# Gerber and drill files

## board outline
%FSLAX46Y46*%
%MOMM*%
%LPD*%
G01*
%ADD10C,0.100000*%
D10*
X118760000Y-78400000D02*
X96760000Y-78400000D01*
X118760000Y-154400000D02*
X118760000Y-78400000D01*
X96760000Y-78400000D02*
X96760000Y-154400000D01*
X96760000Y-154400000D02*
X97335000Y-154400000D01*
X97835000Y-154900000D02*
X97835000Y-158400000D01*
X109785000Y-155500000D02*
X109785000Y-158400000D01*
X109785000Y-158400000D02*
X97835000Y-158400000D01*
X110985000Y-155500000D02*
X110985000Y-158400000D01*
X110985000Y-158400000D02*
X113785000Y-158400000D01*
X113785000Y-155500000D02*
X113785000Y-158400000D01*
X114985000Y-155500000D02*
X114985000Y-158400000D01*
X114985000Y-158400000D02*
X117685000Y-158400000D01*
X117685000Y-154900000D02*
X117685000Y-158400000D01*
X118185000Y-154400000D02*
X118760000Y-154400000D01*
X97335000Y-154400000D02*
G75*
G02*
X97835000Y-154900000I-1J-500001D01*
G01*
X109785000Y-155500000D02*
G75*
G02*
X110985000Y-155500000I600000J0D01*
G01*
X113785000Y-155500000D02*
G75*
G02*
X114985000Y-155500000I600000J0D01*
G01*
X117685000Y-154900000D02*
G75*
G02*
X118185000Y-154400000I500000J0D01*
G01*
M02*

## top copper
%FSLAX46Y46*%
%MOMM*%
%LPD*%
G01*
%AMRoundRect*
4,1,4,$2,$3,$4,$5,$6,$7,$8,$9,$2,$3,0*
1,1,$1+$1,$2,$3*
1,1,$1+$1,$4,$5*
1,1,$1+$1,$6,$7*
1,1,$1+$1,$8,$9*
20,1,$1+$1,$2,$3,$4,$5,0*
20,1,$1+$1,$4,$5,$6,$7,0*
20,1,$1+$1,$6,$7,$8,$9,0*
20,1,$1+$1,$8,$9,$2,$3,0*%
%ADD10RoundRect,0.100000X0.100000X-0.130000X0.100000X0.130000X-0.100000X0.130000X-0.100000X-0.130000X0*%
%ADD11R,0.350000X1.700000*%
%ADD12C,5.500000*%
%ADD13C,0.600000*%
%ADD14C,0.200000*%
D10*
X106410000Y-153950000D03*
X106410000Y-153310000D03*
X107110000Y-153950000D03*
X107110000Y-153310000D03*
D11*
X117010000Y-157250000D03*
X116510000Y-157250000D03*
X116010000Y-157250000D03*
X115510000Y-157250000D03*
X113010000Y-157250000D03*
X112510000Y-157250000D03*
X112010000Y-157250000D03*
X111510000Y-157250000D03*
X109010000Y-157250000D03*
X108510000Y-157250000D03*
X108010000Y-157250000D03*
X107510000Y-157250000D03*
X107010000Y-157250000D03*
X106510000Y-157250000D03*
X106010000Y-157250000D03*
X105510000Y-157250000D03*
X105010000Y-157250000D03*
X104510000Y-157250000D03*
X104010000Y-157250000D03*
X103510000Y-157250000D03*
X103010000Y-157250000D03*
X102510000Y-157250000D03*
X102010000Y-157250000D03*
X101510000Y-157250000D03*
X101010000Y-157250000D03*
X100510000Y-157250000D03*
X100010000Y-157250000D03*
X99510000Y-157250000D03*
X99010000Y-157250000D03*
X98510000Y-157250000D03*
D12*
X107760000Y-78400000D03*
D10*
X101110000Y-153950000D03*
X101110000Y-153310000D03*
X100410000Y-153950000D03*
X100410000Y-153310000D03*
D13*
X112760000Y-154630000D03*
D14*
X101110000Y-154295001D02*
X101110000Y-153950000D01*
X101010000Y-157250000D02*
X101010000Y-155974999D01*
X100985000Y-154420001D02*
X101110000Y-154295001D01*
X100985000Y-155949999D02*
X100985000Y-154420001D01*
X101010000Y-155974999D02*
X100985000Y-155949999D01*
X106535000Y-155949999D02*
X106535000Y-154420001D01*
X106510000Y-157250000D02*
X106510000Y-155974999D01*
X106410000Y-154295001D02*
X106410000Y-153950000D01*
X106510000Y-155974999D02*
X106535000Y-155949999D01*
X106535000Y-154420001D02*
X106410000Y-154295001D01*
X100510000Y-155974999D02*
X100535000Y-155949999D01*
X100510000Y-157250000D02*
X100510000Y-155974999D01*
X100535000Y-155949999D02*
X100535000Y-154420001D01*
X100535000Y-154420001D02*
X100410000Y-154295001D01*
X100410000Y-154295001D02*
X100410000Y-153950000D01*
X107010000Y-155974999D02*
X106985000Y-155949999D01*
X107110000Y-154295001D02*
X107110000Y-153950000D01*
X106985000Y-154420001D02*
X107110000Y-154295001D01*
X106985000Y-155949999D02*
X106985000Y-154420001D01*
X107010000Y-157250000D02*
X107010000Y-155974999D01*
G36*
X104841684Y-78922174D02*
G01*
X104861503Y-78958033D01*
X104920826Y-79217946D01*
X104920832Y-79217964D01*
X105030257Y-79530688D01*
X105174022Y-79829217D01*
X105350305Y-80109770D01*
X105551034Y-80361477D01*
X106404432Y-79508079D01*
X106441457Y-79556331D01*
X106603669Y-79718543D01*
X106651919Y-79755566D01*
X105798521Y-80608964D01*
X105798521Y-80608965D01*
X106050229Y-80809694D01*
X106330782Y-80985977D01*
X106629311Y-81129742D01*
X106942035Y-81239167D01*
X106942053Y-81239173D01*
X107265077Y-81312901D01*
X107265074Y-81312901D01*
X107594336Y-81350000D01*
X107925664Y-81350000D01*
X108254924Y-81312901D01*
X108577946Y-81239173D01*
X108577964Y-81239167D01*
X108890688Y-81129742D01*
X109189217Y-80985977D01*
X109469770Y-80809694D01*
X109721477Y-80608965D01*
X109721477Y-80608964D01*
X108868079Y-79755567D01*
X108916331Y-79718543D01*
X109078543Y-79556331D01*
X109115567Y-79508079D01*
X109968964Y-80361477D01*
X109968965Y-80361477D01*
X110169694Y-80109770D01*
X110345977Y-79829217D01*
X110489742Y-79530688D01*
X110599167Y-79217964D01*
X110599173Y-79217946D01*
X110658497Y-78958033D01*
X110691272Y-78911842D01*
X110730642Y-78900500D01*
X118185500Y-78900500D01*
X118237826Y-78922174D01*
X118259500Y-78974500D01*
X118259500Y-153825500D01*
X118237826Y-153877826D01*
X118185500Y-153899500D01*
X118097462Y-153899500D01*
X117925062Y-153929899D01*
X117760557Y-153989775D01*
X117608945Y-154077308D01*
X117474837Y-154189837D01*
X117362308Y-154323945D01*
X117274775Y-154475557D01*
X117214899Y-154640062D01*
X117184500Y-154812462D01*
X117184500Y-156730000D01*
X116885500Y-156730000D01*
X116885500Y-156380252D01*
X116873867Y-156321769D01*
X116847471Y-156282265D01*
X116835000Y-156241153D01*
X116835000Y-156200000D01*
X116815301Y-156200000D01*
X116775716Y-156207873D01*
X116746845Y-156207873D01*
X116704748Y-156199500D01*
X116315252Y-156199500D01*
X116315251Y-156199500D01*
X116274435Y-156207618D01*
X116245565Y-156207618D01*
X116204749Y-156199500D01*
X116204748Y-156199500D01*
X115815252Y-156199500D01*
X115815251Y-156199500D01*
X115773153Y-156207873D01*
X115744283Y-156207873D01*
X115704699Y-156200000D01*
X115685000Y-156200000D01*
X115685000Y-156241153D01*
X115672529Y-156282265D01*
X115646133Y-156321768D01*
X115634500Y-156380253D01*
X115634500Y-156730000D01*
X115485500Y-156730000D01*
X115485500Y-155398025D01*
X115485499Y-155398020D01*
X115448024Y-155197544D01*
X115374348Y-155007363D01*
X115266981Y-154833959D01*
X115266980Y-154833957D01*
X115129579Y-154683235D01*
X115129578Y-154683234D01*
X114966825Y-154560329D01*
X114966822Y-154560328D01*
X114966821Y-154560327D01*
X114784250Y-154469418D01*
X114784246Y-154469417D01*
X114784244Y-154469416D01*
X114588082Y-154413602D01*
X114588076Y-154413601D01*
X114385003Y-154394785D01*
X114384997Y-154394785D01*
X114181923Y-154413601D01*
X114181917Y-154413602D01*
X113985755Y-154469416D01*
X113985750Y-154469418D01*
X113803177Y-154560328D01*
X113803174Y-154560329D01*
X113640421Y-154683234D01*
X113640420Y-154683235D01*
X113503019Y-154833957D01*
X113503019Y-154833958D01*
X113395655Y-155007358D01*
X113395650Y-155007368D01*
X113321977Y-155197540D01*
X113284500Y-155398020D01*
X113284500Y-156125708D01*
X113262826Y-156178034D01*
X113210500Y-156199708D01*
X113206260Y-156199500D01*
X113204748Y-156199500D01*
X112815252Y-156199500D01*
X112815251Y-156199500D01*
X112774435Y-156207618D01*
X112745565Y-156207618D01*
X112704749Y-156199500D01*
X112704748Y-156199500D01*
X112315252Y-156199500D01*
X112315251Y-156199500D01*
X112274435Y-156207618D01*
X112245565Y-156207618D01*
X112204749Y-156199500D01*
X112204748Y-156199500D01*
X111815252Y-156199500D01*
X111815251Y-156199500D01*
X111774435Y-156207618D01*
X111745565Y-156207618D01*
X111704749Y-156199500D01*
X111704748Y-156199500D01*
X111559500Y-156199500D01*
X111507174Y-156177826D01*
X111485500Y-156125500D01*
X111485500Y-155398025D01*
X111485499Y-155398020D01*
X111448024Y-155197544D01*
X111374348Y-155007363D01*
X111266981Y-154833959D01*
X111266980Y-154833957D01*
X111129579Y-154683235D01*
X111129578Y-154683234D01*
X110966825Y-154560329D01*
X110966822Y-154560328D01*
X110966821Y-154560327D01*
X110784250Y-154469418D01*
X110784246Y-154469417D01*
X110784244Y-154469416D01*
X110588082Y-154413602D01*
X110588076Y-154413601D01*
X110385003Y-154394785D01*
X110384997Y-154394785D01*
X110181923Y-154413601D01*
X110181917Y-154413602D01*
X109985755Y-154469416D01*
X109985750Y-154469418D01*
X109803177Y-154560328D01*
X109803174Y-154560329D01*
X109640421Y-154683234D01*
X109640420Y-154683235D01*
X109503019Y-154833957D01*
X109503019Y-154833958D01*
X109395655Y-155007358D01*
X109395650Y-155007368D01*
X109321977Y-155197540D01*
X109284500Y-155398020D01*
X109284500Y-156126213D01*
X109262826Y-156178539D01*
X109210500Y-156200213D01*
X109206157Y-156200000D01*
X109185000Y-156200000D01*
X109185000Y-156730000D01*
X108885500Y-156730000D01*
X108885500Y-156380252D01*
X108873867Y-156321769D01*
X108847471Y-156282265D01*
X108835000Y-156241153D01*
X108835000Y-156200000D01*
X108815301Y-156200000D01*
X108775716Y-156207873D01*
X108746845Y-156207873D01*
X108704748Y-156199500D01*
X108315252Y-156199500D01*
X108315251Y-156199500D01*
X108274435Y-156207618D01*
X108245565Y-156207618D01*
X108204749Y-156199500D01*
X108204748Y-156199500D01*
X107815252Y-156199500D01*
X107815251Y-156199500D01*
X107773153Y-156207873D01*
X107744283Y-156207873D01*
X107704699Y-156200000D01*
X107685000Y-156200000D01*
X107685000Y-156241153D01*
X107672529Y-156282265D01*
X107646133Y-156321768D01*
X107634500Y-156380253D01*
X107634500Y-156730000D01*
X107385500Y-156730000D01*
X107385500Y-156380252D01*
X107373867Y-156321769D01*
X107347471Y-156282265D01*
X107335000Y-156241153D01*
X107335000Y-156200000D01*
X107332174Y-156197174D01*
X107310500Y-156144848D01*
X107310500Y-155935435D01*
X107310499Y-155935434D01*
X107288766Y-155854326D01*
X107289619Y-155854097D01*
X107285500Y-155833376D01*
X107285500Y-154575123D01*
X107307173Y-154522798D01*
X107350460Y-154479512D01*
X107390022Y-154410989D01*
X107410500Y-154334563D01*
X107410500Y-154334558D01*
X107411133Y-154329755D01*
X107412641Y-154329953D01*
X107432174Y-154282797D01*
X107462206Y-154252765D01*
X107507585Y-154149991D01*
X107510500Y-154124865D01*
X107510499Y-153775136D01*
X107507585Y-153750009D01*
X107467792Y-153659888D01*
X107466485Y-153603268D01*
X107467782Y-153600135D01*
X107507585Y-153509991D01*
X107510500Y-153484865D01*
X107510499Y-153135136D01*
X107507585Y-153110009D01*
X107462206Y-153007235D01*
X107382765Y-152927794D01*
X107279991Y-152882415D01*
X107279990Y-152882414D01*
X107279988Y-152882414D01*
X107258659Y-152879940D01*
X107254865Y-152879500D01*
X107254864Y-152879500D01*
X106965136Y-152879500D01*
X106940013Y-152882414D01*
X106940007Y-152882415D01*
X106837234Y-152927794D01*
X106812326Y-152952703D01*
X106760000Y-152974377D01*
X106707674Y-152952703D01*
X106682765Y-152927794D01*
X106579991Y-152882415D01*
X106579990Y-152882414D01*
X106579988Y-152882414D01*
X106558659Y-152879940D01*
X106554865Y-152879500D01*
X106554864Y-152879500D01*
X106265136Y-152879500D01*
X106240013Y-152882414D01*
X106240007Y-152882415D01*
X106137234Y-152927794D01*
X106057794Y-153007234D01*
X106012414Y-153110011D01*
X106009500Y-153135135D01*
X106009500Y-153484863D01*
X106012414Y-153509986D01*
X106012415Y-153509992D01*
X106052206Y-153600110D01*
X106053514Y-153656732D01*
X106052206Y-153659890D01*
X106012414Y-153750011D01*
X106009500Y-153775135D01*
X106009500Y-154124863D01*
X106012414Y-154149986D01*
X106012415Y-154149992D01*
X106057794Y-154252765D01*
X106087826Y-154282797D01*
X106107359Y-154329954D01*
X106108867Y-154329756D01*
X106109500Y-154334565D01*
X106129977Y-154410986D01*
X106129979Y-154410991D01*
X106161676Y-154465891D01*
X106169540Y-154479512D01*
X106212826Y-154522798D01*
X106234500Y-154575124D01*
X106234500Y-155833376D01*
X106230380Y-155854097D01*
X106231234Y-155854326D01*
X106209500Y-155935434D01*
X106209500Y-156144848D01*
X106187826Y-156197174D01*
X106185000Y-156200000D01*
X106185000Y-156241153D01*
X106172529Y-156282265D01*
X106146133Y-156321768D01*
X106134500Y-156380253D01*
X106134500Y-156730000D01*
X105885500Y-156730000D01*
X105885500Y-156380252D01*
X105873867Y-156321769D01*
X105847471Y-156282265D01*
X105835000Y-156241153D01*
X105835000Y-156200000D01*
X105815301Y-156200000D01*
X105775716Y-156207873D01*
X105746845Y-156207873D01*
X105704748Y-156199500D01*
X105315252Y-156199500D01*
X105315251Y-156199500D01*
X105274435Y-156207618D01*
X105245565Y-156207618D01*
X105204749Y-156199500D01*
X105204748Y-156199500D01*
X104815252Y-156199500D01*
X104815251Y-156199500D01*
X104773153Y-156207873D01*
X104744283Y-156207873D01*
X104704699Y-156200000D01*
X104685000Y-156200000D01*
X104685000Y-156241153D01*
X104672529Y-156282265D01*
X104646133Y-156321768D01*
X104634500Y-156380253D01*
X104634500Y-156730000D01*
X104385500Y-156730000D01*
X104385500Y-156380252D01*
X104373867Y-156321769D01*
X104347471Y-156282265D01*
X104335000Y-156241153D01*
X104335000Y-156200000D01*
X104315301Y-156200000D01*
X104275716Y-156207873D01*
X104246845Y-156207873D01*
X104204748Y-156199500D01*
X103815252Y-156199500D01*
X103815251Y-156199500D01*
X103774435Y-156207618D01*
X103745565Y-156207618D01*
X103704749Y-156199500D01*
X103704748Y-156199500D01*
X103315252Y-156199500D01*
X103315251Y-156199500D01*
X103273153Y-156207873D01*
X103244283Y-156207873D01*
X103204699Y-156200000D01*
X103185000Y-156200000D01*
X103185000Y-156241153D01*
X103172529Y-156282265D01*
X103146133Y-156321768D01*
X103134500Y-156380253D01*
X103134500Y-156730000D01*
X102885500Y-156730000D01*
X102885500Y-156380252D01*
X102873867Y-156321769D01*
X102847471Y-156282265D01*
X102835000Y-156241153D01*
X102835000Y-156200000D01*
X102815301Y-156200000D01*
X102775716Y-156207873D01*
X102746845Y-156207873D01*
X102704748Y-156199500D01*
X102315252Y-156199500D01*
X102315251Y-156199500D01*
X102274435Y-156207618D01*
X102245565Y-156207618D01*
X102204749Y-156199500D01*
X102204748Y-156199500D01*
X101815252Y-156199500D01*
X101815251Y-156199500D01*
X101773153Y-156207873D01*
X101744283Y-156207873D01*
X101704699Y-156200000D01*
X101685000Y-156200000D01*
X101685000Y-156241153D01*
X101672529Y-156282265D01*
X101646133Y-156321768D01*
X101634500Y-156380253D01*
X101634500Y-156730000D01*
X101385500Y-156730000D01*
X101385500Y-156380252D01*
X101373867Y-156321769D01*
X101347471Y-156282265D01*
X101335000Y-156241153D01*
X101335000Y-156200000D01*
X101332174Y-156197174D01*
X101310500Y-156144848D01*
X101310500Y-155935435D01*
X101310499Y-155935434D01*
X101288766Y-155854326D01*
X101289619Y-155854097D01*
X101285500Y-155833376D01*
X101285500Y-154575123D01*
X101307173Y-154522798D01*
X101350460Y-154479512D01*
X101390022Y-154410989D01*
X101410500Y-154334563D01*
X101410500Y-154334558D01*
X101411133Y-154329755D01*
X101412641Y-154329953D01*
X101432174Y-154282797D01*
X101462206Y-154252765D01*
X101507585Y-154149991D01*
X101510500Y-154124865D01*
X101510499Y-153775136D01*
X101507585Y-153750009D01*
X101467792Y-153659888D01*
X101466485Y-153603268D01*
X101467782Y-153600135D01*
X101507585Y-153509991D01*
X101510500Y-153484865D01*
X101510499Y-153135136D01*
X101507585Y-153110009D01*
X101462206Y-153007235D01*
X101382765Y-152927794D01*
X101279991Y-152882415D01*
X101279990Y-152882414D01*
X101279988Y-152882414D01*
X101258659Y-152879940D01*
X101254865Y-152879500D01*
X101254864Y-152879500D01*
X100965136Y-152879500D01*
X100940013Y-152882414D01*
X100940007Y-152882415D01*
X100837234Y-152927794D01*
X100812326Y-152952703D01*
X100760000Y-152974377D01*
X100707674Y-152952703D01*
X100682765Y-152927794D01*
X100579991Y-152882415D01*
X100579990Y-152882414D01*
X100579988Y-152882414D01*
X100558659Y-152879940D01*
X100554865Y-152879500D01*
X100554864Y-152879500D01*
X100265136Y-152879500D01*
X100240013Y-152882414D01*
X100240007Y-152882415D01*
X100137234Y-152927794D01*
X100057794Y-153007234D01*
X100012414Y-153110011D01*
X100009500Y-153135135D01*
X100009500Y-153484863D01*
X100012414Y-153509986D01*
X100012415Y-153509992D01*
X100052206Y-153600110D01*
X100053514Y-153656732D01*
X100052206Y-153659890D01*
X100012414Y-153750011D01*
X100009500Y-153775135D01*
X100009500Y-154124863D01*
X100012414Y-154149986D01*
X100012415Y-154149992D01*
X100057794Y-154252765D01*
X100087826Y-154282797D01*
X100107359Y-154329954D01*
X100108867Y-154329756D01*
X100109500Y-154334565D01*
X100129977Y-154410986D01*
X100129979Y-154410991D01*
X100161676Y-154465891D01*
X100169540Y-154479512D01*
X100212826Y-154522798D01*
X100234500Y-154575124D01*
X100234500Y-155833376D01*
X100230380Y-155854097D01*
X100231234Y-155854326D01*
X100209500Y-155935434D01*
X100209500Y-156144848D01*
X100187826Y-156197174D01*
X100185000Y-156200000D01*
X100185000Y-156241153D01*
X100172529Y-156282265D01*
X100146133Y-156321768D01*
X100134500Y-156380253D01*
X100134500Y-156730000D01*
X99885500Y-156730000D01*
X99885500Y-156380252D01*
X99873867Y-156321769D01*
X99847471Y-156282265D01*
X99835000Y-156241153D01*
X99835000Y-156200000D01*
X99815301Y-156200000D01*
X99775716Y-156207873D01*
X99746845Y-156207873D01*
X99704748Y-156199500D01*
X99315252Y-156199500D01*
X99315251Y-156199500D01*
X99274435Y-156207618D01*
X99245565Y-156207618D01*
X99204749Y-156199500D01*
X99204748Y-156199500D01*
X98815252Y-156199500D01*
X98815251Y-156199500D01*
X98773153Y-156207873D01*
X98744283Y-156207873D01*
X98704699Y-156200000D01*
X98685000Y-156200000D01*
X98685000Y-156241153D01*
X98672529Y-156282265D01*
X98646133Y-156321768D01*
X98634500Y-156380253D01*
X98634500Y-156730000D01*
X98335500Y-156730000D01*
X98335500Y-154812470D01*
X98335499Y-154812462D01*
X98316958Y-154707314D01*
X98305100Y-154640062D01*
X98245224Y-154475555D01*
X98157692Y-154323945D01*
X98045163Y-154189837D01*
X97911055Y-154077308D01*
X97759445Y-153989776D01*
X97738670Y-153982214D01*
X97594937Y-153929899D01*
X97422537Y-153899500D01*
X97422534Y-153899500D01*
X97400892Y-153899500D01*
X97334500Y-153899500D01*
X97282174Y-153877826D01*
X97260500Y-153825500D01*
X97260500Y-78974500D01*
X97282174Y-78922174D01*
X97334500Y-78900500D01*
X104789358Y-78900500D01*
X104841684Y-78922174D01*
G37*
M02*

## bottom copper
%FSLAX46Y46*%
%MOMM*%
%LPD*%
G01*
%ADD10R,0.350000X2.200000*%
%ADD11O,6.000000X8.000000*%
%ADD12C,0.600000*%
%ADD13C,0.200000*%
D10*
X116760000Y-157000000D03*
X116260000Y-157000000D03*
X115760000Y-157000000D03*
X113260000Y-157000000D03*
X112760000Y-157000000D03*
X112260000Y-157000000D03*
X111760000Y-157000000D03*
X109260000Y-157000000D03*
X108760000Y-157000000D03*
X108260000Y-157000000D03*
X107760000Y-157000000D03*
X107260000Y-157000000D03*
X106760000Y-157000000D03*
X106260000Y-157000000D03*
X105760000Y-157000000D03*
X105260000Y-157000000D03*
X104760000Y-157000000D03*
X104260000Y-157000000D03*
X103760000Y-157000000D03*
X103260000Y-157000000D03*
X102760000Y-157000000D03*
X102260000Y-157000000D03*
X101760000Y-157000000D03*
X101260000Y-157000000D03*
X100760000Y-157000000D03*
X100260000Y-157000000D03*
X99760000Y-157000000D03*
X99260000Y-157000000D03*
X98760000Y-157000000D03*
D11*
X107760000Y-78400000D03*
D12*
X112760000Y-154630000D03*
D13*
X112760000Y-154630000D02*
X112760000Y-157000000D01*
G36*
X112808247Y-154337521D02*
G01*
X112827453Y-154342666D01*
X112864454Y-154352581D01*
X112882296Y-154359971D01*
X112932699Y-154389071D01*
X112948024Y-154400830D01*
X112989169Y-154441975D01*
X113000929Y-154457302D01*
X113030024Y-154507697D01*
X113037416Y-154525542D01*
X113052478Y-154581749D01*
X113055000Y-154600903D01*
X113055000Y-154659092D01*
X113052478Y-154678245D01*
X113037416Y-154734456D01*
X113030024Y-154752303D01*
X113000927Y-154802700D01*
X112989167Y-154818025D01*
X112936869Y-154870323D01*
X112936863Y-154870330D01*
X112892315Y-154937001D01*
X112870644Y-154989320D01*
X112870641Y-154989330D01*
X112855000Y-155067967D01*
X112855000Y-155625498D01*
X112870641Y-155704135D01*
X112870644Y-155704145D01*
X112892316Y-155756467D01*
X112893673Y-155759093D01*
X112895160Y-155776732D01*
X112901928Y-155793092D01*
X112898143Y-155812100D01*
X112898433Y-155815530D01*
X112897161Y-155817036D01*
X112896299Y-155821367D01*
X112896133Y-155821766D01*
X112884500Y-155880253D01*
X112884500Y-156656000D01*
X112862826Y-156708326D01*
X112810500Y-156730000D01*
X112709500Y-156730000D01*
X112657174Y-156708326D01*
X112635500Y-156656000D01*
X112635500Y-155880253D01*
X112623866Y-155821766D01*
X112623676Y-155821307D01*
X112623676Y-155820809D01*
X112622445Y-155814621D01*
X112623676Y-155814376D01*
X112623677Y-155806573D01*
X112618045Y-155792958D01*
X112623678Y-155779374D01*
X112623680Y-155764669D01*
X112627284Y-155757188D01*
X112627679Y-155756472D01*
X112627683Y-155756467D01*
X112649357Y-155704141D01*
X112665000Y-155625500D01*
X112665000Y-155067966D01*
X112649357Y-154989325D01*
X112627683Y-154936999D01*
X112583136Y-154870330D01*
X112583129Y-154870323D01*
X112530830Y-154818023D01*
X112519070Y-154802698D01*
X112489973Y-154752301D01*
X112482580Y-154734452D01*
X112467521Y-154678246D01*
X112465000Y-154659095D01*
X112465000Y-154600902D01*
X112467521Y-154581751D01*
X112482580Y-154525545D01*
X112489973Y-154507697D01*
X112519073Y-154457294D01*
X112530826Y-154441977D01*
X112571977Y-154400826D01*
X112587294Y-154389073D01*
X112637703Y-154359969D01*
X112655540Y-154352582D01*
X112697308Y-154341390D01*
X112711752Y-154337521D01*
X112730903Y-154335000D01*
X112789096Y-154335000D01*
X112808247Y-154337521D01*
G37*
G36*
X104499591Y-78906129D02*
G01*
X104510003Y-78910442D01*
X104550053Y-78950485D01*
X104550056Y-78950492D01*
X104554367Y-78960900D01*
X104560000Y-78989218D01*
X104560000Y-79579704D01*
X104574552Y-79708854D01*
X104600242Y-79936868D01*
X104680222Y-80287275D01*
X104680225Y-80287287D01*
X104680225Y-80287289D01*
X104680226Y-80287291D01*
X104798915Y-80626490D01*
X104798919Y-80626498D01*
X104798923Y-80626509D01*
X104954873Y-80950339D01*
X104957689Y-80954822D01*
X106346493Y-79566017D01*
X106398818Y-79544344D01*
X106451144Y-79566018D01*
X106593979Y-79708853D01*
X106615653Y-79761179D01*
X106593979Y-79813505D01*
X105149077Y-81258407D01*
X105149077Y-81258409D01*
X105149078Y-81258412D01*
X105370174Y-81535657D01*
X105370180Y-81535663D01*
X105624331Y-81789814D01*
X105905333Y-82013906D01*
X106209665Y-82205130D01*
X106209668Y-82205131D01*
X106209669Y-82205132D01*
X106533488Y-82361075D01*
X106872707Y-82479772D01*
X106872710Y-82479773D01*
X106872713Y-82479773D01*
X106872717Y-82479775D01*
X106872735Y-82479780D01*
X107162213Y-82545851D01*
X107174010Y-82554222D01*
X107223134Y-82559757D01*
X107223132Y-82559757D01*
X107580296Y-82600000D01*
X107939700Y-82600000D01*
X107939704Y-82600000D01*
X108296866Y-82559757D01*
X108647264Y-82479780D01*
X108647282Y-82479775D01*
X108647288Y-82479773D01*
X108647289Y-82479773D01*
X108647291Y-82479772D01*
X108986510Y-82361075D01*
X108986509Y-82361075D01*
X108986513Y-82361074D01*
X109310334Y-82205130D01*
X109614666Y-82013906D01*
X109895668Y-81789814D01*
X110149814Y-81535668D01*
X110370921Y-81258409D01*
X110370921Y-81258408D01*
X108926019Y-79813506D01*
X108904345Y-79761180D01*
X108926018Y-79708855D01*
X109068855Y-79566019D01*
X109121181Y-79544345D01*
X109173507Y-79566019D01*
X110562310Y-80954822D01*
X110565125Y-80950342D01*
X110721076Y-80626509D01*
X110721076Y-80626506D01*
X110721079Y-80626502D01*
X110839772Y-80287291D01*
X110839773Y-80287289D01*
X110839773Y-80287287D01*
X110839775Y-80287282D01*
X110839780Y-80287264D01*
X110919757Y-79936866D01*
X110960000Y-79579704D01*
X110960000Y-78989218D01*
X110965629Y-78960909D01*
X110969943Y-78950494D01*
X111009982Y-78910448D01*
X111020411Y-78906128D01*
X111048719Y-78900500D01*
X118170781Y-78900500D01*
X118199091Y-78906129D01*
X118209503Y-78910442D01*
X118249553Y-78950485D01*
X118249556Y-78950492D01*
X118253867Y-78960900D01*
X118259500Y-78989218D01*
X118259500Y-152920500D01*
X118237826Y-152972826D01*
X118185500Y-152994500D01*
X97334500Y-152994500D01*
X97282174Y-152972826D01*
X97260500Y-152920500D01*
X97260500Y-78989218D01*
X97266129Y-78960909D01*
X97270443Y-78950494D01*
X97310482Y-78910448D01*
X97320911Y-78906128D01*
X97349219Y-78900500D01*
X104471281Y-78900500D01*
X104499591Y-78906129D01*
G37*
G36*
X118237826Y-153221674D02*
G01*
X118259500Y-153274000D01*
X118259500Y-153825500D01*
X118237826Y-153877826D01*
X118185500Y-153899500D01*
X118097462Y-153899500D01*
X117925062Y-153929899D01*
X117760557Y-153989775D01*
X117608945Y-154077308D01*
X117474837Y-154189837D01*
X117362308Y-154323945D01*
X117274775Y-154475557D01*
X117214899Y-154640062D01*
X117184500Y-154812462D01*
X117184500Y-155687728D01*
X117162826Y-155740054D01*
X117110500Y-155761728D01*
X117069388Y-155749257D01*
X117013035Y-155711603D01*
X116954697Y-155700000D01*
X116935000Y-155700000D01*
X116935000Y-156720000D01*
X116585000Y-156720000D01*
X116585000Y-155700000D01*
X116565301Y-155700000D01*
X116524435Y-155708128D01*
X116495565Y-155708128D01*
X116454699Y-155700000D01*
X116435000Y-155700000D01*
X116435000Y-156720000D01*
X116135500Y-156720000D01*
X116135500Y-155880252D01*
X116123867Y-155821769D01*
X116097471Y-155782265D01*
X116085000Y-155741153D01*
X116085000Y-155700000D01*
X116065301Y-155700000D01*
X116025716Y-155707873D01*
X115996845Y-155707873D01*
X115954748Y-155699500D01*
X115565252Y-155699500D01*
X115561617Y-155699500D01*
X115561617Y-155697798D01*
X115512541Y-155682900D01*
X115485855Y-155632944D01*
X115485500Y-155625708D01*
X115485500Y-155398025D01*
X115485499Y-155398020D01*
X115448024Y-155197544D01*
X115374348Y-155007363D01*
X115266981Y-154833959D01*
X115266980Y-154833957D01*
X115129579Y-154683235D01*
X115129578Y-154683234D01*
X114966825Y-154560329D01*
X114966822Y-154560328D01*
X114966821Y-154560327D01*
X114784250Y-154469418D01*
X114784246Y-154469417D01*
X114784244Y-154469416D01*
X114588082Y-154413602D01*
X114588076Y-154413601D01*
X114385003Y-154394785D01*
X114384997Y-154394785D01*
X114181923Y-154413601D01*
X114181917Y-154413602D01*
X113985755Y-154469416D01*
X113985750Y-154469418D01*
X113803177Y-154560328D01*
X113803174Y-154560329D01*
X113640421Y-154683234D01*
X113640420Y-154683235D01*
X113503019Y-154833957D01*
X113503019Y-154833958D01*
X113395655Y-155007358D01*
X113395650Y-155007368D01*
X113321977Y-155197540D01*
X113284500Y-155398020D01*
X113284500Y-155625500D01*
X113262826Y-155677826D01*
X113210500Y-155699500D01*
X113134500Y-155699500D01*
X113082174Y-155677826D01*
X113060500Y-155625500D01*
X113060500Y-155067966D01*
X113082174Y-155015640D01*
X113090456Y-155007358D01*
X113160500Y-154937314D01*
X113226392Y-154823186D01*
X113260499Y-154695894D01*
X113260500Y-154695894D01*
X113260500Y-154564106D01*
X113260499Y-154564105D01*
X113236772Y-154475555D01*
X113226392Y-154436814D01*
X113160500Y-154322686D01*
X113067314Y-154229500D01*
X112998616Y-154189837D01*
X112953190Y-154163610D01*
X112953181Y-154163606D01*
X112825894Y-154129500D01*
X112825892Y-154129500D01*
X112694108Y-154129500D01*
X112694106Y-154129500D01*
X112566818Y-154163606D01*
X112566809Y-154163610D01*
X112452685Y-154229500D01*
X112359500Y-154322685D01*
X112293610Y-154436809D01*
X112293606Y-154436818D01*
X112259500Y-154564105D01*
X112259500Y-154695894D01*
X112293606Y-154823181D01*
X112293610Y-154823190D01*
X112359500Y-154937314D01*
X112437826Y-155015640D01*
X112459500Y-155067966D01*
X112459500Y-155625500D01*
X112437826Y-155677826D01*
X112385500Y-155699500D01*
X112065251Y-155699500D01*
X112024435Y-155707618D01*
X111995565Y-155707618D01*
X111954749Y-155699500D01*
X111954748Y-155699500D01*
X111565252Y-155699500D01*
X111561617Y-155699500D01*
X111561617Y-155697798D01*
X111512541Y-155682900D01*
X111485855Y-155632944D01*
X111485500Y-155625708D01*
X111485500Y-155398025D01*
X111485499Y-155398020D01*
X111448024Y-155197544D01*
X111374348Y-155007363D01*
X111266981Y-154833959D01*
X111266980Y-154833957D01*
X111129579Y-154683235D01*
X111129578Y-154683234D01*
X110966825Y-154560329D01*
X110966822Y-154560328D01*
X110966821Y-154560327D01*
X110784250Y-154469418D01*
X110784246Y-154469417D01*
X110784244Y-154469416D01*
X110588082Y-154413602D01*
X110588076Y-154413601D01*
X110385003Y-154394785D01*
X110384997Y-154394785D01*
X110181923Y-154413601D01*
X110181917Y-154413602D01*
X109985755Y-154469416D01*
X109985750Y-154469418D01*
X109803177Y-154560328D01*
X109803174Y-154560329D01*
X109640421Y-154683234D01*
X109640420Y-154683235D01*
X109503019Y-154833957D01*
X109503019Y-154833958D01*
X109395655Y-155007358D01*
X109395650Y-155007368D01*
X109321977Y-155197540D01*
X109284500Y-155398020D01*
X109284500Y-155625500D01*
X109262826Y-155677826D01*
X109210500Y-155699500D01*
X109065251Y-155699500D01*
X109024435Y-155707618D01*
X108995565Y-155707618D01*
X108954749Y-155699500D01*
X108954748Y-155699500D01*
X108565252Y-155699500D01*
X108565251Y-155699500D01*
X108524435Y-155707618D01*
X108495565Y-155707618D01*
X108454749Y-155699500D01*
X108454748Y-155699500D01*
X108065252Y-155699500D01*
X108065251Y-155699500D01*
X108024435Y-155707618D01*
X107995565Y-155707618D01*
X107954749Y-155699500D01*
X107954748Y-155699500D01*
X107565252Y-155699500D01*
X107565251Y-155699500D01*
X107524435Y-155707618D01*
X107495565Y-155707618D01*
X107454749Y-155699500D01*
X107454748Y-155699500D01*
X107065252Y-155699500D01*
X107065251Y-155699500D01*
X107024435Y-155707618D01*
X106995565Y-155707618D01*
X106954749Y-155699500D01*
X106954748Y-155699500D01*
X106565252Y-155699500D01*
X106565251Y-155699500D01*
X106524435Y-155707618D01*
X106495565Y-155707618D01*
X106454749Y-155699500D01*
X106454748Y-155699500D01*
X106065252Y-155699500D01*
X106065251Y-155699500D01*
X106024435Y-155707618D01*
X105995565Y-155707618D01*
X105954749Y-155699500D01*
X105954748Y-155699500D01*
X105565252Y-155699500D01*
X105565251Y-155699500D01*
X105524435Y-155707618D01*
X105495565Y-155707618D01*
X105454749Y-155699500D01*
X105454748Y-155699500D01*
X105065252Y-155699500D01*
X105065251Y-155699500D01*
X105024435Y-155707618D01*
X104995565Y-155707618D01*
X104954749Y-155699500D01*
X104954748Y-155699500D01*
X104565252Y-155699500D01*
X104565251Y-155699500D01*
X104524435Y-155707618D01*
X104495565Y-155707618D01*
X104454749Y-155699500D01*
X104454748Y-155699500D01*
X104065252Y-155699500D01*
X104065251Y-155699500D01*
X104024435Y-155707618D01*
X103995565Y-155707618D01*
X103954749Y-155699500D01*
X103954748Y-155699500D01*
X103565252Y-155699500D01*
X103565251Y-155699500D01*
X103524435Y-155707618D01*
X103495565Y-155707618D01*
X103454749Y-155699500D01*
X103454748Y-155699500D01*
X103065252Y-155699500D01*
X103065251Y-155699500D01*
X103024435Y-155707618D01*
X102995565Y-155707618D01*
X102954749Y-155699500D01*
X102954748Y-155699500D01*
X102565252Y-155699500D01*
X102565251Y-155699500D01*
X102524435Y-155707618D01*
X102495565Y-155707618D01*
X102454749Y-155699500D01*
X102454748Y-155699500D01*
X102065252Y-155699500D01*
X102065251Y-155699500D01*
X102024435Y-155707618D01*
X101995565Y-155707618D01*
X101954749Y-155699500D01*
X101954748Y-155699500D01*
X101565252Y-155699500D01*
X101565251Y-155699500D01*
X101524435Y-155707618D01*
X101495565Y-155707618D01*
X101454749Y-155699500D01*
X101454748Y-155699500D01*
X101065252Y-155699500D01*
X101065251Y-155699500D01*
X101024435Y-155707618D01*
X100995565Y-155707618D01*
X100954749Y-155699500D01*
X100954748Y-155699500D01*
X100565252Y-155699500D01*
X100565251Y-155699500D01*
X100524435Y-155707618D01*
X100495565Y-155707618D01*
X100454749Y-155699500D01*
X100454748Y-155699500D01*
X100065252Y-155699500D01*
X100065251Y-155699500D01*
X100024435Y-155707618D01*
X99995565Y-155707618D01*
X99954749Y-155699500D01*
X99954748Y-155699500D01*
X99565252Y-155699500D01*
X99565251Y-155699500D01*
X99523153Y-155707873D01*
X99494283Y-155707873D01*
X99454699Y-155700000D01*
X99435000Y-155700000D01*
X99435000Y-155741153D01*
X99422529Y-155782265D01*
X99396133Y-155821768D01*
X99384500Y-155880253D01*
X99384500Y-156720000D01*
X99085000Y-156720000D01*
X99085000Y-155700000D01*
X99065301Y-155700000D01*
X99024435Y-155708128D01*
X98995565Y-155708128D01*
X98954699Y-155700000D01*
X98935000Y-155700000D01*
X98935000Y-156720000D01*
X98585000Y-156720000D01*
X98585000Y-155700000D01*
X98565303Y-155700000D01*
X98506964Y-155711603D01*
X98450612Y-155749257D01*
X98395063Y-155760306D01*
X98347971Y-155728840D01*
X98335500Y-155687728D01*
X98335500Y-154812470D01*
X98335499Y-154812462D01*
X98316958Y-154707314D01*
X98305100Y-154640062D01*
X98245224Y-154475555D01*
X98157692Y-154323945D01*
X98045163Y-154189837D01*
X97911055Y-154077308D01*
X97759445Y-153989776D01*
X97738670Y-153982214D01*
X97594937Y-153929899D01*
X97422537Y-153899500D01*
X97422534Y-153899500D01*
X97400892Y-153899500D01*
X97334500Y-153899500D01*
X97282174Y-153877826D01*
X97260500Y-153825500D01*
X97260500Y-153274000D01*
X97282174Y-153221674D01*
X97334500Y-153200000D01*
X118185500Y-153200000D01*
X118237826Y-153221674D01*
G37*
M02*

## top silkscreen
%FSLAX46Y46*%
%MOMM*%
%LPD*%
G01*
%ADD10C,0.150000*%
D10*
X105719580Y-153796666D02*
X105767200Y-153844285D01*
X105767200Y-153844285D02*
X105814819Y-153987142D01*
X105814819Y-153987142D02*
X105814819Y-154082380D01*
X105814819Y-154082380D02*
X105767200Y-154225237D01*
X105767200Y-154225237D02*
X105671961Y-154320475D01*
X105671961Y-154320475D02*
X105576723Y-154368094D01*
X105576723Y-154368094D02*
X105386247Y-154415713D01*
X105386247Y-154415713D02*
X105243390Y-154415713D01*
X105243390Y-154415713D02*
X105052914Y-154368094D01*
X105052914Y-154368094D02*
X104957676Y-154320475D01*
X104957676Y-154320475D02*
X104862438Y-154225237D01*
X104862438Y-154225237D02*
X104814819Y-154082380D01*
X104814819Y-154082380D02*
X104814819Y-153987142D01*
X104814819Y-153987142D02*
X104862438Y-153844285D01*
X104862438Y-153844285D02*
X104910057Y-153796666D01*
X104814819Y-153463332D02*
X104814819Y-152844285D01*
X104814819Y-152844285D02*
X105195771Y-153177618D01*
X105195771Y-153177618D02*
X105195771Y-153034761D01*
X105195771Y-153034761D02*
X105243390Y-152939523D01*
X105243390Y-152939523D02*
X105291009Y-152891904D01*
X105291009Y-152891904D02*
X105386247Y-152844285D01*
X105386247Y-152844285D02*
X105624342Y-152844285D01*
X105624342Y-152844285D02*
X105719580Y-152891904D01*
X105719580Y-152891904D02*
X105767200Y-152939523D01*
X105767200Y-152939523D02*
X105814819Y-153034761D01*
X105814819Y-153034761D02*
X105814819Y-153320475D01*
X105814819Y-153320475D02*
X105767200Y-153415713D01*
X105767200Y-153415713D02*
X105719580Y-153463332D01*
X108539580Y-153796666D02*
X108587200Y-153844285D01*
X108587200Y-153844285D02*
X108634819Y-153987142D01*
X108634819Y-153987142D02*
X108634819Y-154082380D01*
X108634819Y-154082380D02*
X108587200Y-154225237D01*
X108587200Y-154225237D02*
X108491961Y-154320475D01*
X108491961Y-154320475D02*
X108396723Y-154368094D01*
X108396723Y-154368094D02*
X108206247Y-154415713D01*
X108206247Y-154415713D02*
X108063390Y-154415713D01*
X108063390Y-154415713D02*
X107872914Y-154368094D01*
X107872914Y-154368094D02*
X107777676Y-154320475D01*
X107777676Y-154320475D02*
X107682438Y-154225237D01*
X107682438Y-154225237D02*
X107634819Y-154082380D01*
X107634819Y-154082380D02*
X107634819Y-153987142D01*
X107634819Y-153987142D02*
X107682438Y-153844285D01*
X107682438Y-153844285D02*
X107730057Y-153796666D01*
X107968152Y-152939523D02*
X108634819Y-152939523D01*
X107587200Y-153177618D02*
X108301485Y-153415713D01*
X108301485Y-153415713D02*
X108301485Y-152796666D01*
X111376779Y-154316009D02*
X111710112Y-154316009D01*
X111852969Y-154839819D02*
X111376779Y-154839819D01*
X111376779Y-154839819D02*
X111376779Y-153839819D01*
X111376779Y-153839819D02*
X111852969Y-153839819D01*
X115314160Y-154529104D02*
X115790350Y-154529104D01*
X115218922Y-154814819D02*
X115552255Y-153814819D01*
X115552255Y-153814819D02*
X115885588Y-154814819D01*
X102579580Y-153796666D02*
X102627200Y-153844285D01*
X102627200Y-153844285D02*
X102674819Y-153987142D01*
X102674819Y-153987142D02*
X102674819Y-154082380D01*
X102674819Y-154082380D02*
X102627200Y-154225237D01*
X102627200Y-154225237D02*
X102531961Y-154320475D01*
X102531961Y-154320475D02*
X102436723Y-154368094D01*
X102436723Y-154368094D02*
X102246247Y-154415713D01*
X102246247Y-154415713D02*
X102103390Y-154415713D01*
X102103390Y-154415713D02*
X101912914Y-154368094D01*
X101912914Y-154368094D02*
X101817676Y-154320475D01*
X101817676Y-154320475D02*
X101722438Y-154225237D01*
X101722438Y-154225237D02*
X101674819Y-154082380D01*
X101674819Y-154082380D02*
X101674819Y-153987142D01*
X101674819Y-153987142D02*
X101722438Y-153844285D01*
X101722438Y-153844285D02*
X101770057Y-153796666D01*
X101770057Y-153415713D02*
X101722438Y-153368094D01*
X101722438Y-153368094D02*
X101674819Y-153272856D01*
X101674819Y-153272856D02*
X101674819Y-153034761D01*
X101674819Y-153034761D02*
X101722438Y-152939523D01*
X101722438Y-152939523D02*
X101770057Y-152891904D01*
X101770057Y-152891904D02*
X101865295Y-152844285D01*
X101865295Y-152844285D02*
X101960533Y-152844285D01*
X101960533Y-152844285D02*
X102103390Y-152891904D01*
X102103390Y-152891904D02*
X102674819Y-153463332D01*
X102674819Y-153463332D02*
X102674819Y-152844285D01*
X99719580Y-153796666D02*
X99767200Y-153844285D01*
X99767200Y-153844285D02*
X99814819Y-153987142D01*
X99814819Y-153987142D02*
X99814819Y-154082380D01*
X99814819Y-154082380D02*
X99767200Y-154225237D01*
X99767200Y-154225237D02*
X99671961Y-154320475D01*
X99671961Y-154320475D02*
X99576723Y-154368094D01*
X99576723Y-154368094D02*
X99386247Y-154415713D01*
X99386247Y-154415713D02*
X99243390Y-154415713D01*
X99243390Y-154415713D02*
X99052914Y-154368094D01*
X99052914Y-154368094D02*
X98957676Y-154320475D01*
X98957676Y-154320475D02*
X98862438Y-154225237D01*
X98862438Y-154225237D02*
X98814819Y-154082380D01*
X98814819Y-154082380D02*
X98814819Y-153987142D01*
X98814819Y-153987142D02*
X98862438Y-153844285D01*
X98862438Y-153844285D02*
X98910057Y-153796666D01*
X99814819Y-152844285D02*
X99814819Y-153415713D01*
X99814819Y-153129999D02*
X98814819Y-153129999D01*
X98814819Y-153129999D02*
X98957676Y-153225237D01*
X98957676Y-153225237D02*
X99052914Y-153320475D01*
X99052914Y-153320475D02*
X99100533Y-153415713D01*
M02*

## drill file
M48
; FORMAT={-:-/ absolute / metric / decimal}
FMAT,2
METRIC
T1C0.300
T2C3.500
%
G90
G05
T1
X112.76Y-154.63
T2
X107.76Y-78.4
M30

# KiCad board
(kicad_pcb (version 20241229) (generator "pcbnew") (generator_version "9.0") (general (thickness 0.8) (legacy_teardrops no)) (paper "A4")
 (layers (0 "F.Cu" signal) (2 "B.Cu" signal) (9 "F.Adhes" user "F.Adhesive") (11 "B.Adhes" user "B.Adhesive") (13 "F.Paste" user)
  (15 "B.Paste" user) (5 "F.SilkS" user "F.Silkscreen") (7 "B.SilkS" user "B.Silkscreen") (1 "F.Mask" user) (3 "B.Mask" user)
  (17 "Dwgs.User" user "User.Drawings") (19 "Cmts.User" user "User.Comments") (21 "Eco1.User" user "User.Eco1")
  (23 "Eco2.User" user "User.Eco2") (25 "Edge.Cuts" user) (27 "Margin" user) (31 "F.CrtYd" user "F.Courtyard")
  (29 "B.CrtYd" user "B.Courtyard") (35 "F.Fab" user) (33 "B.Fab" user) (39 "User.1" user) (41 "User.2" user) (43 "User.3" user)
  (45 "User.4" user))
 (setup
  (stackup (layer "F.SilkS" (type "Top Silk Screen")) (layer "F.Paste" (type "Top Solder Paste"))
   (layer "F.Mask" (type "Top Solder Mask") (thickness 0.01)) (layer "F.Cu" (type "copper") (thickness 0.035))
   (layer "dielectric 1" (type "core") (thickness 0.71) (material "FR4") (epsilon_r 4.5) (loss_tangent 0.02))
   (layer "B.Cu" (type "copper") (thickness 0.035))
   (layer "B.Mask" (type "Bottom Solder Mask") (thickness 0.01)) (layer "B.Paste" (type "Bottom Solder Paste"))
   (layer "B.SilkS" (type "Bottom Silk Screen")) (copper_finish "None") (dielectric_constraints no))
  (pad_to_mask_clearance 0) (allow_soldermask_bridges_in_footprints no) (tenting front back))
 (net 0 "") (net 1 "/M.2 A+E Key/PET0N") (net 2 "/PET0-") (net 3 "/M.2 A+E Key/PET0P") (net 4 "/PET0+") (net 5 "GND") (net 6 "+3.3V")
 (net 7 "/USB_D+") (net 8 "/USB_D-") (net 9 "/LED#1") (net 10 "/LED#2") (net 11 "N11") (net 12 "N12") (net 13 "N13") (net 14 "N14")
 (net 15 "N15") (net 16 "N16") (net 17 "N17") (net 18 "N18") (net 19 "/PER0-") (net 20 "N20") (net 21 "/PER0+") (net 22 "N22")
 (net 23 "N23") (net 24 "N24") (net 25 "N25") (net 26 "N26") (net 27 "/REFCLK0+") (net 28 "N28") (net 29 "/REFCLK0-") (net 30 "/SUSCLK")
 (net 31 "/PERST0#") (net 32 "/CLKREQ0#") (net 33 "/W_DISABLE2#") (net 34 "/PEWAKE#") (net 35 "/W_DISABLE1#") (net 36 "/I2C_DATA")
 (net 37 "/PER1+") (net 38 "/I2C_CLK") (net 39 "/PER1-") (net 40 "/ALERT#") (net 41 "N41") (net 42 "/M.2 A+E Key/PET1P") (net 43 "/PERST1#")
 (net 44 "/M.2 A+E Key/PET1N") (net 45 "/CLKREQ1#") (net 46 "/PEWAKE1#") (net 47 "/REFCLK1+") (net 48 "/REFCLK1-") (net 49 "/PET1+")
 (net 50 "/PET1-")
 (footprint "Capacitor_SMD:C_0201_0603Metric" (layer "F.Cu") (at 106.41 153.63 90)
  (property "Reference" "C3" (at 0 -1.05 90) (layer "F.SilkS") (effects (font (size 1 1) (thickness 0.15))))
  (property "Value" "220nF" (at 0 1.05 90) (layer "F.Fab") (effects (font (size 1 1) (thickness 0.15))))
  (pad "" smd roundrect (at -0.345 0 90) (size 0.318 0.36) (layers "F.Paste") (roundrect_rratio 0.25))
  (pad "" smd roundrect (at 0.345 0 90) (size 0.318 0.36) (layers "F.Paste") (roundrect_rratio 0.25))
  (pad "1" smd roundrect (at -0.32 0 90) (size 0.46 0.4) (layers "F.Cu" "F.Mask") (roundrect_rratio 0.25) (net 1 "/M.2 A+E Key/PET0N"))
  (pad "2" smd roundrect (at 0.32 0 90) (size 0.46 0.4) (layers "F.Cu" "F.Mask") (roundrect_rratio 0.25) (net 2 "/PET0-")))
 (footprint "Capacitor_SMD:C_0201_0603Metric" (layer "F.Cu") (at 107.11 153.63 90)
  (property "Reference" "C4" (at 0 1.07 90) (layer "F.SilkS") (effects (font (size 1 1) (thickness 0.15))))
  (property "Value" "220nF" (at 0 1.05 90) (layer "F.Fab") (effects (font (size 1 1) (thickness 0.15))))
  (pad "" smd roundrect (at -0.345 0 90) (size 0.318 0.36) (layers "F.Paste") (roundrect_rratio 0.25))
  (pad "" smd roundrect (at 0.345 0 90) (size 0.318 0.36) (layers "F.Paste") (roundrect_rratio 0.25))
  (pad "1" smd roundrect (at -0.32 0 90) (size 0.46 0.4) (layers "F.Cu" "F.Mask") (roundrect_rratio 0.25) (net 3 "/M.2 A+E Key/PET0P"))
  (pad "2" smd roundrect (at 0.32 0 90) (size 0.46 0.4) (layers "F.Cu" "F.Mask") (roundrect_rratio 0.25) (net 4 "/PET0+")))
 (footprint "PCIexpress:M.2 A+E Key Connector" (layer "F.Cu") (at 107.76 157.29)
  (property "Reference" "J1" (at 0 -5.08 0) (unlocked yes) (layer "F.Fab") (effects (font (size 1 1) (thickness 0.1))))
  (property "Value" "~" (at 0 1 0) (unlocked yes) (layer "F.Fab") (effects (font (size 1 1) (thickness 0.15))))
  (fp_line (start -11 -2.89) (end -10.425 -2.89) (stroke (width 0.1) (type default)) (layer "Edge.Cuts"))
  (fp_line (start -9.925 -2.39) (end -9.925 1.11) (stroke (width 0.1) (type default)) (layer "Edge.Cuts"))
  (fp_line (start 2.025 -1.79) (end 2.025 1.11) (stroke (width 0.1) (type default)) (layer "Edge.Cuts"))
  (fp_line (start 2.025 1.11) (end -9.925 1.11) (stroke (width 0.1) (type default)) (layer "Edge.Cuts"))
  (fp_line (start 3.225 -1.79) (end 3.225 1.11) (stroke (width 0.1) (type default)) (layer "Edge.Cuts"))
  (fp_line (start 3.225 1.11) (end 6.025 1.11) (stroke (width 0.1) (type default)) (layer "Edge.Cuts"))
  (fp_line (start 6.025 -1.79) (end 6.025 1.11) (stroke (width 0.1) (type default)) (layer "Edge.Cuts"))
  (fp_line (start 7.225 -1.79) (end 7.225 1.11) (stroke (width 0.1) (type default)) (layer "Edge.Cuts"))
  (fp_line (start 7.225 1.11) (end 9.925 1.11) (stroke (width 0.1) (type default)) (layer "Edge.Cuts"))
  (fp_line (start 9.925 -2.39) (end 9.925 1.11) (stroke (width 0.1) (type default)) (layer "Edge.Cuts"))
  (fp_line (start 10.425 -2.89) (end 11 -2.89) (stroke (width 0.1) (type default)) (layer "Edge.Cuts"))
  (fp_arc (start -10.425 -2.89) (mid -10.071447 -2.743553) (end -9.925 -2.39) (stroke (width 0.1) (type default)) (layer "Edge.Cuts"))
  (fp_arc (start 2.025 -1.79) (mid 2.625 -2.39) (end 3.225 -1.79) (stroke (width 0.1) (type default)) (layer "Edge.Cuts"))
  (fp_arc (start 6.025 -1.79) (mid 6.625 -2.39) (end 7.225 -1.79) (stroke (width 0.1) (type default)) (layer "Edge.Cuts"))
  (fp_arc (start 9.925 -2.39) (mid 10.071447 -2.743553) (end 10.425 -2.89) (stroke (width 0.1) (type default)) (layer "Edge.Cuts"))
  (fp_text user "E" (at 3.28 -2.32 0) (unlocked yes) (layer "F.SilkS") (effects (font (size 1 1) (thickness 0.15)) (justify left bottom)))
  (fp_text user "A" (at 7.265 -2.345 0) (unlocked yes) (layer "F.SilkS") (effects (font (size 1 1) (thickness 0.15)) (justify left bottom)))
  (pad "1" smd rect (at 9.25 -0.04 180) (size 0.35 1.7) (layers "F.Cu") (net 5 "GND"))
  (pad "2" smd rect (at 9 -0.29 180) (size 0.35 2.2) (layers "B.Cu") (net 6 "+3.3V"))
  (pad "3" smd rect (at 8.75 -0.04 180) (size 0.35 1.7) (layers "F.Cu") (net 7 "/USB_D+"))
  (pad "4" smd rect (at 8.5 -0.29 180) (size 0.35 2.2) (layers "B.Cu") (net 6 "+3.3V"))
  (pad "5" smd rect (at 8.25 -0.04 180) (size 0.35 1.7) (layers "F.Cu") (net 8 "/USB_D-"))
  (pad "6" smd rect (at 8 -0.29 180) (size 0.35 2.2) (layers "B.Cu") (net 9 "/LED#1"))
  (pad "7" smd rect (at 7.75 -0.04 180) (size 0.35 1.7) (layers "F.Cu") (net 5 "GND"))
  (pad "16" smd rect (at 5.5 -0.29 180) (size 0.35 2.2) (layers "B.Cu") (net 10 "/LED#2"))
  (pad "17" smd rect (at 5.25 -0.04 180) (size 0.35 1.7) (layers "F.Cu") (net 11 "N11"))
  (pad "18" smd rect (at 5 -0.29 180) (size 0.35 2.2) (layers "B.Cu") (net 5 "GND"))
  (pad "19" smd rect (at 4.75 -0.04 180) (size 0.35 1.7) (layers "F.Cu") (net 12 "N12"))
  (pad "20" smd rect (at 4.5 -0.29 180) (size 0.35 2.2) (layers "B.Cu") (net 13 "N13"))
  (pad "21" smd rect (at 4.25 -0.04 180) (size 0.35 1.7) (layers "F.Cu") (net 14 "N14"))
  (pad "22" smd rect (at 4 -0.29 180) (size 0.35 2.2) (layers "B.Cu") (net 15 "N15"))
  (pad "23" smd rect (at 3.75 -0.04 180) (size 0.35 1.7) (layers "F.Cu") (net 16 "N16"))
  (pad "32" smd rect (at 1.5 -0.29 180) (size 0.35 2.2) (layers "B.Cu") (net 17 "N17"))
  (pad "33" smd rect (at 1.25 -0.04 180) (size 0.35 1.7) (layers "F.Cu") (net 5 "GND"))
  (pad "34" smd rect (at 1 -0.29 180) (size 0.35 2.2) (layers "B.Cu") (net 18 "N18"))
  (pad "35" smd rect (at 0.75 -0.04 180) (size 0.35 1.7) (layers "F.Cu") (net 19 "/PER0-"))
  (pad "36" smd rect (at 0.5 -0.29 180) (size 0.35 2.2) (layers "B.Cu") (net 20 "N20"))
  (pad "37" smd rect (at 0.25 -0.04 180) (size 0.35 1.7) (layers "F.Cu") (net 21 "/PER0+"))
  (pad "38" smd rect (at 0 -0.29 180) (size 0.35 2.2) (layers "B.Cu") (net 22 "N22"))
  (pad "39" smd rect (at -0.25 -0.04 180) (size 0.35 1.7) (layers "F.Cu") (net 5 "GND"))
  (pad "40" smd rect (at -0.5 -0.29 180) (size 0.35 2.2) (layers "B.Cu") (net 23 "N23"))
  (pad "41" smd rect (at -0.75 -0.04 180) (size 0.35 1.7) (layers "F.Cu") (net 3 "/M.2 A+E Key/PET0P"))
  (pad "42" smd rect (at -1 -0.29 180) (size 0.35 2.2) (layers "B.Cu") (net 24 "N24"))
  (pad "43" smd rect (at -1.25 -0.04 180) (size 0.35 1.7) (layers "F.Cu") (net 1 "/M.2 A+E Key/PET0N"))
  (pad "44" smd rect (at -1.5 -0.29 180) (size 0.35 2.2) (layers "B.Cu") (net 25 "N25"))
  (pad "45" smd rect (at -1.75 -0.04 180) (size 0.35 1.7) (layers "F.Cu") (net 5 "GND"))
  (pad "46" smd rect (at -2 -0.29 180) (size 0.35 2.2) (layers "B.Cu") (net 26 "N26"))
  (pad "47" smd rect (at -2.25 -0.04 180) (size 0.35 1.7) (layers "F.Cu") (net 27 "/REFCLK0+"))
  (pad "48" smd rect (at -2.5 -0.29 180) (size 0.35 2.2) (layers "B.Cu") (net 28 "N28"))
  (pad "49" smd rect (at -2.75 -0.04 180) (size 0.35 1.7) (layers "F.Cu") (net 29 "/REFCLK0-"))
  (pad "50" smd rect (at -3 -0.29 180) (size 0.35 2.2) (layers "B.Cu") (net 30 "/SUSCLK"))
  (pad "51" smd rect (at -3.25 -0.04 180) (size 0.35 1.7) (layers "F.Cu") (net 5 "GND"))
  (pad "52" smd rect (at -3.5 -0.29 180) (size 0.35 2.2) (layers "B.Cu") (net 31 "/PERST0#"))
  (pad "53" smd rect (at -3.75 -0.04 180) (size 0.35 1.7) (layers "F.Cu") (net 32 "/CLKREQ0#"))
  (pad "54" smd rect (at -4 -0.29 180) (size 0.35 2.2) (layers "B.Cu") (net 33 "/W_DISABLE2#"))
  (pad "55" smd rect (at -4.25 -0.04 180) (size 0.35 1.7) (layers "F.Cu") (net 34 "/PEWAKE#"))
  (pad "56" smd rect (at -4.5 -0.29 180) (size 0.35 2.2) (layers "B.Cu") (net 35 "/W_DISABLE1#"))
  (pad "57" smd rect (at -4.75 -0.04 180) (size 0.35 1.7) (layers "F.Cu") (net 5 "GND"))
  (pad "58" smd rect (at -5 -0.29 180) (size 0.35 2.2) (layers "B.Cu") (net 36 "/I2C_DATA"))
  (pad "59" smd rect (at -5.25 -0.04 180) (size 0.35 1.7) (layers "F.Cu") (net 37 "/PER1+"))
  (pad "60" smd rect (at -5.5 -0.29 180) (size 0.35 2.2) (layers "B.Cu") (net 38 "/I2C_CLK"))
  (pad "61" smd rect (at -5.75 -0.04 180) (size 0.35 1.7) (layers "F.Cu") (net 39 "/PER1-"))
  (pad "62" smd rect (at -6 -0.29 180) (size 0.35 2.2) (layers "B.Cu") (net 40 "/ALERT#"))
  (pad "63" smd rect (at -6.25 -0.04 180) (size 0.35 1.7) (layers "F.Cu") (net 5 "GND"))
  (pad "64" smd rect (at -6.5 -0.29 180) (size 0.35 2.2) (layers "B.Cu") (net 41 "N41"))
  (pad "65" smd rect (at -6.75 -0.04 180) (size 0.35 1.7) (layers "F.Cu") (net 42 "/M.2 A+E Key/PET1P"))
  (pad "66" smd rect (at -7 -0.29 180) (size 0.35 2.2) (layers "B.Cu") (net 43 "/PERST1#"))
  (pad "67" smd rect (at -7.25 -0.04 180) (size 0.35 1.7) (layers "F.Cu") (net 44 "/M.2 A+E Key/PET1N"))
  (pad "68" smd rect (at -7.5 -0.29 180) (size 0.35 2.2) (layers "B.Cu") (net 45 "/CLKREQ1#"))
  (pad "69" smd rect (at -7.75 -0.04 180) (size 0.35 1.7) (layers "F.Cu") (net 5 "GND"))
  (pad "70" smd rect (at -8 -0.29 180) (size 0.35 2.2) (layers "B.Cu") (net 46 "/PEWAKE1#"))
  (pad "71" smd rect (at -8.25 -0.04 180) (size 0.35 1.7) (layers "F.Cu") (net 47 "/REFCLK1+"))
  (pad "72" smd rect (at -8.5 -0.29 180) (size 0.35 2.2) (layers "B.Cu") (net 6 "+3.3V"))
  (pad "73" smd rect (at -8.75 -0.04 180) (size 0.35 1.7) (layers "F.Cu") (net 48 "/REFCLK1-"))
  (pad "74" smd rect (at -9 -0.29 180) (size 0.35 2.2) (layers "B.Cu") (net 6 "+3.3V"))
  (pad "75" smd rect (at -9.25 -0.04 180) (size 0.35 1.7) (layers "F.Cu") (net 5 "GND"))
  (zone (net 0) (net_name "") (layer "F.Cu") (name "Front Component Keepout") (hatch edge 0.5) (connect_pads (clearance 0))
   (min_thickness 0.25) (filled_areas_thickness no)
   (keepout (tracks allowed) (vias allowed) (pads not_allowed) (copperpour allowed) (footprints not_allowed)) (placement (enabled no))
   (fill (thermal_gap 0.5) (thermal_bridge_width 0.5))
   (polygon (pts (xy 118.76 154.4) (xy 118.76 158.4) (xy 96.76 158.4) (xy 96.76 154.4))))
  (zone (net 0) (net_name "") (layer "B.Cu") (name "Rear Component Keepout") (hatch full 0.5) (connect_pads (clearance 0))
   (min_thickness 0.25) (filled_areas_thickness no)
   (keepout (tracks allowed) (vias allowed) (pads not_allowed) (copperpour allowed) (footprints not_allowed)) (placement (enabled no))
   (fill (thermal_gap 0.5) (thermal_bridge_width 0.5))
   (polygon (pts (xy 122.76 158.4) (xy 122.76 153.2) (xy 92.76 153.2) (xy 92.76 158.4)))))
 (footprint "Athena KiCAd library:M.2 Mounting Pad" (layer "F.Cu") (at 107.76 78.4)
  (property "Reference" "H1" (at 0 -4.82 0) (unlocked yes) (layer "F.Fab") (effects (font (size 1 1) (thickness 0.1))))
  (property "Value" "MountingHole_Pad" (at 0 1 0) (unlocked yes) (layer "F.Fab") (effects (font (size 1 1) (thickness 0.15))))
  (pad "1" thru_hole circle (at 0 0) (size 5.5 5.5) (drill 3.5) (layers "*.Cu" "*.Mask") (remove_unused_layers no) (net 5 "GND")
   (padstack (mode front_inner_back)
    (layer "Inner" (shape circle) (size 5.5 5.5) (zone_connect -1))
    (layer "B.Cu" (shape oval) (size 6 8) (thermal_bridge_angle 45) (zone_connect -1)))))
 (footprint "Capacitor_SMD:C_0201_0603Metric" (layer "F.Cu") (at 101.11 153.63 90)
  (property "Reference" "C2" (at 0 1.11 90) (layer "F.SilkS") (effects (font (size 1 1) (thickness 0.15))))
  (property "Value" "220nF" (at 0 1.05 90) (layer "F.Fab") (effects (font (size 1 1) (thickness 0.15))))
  (pad "" smd roundrect (at -0.345 0 90) (size 0.318 0.36) (layers "F.Paste") (roundrect_rratio 0.25))
  (pad "" smd roundrect (at 0.345 0 90) (size 0.318 0.36) (layers "F.Paste") (roundrect_rratio 0.25))
  (pad "1" smd roundrect (at -0.32 0 90) (size 0.46 0.4) (layers "F.Cu" "F.Mask") (roundrect_rratio 0.25) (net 42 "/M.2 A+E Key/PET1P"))
  (pad "2" smd roundrect (at 0.32 0 90) (size 0.46 0.4) (layers "F.Cu" "F.Mask") (roundrect_rratio 0.25) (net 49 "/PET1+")))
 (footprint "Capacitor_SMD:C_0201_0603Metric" (layer "F.Cu") (at 100.41 153.63 90)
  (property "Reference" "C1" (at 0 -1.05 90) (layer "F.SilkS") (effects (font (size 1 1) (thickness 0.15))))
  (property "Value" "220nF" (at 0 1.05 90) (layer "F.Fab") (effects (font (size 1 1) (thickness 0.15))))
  (pad "" smd roundrect (at -0.345 0 90) (size 0.318 0.36) (layers "F.Paste") (roundrect_rratio 0.25))
  (pad "" smd roundrect (at 0.345 0 90) (size 0.318 0.36) (layers "F.Paste") (roundrect_rratio 0.25))
  (pad "1" smd roundrect (at -0.32 0 90) (size 0.46 0.4) (layers "F.Cu" "F.Mask") (roundrect_rratio 0.25) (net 44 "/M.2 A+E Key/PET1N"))
  (pad "2" smd roundrect (at 0.32 0 90) (size 0.46 0.4) (layers "F.Cu" "F.Mask") (roundrect_rratio 0.25) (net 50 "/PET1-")))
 (gr_line (start 118.76 78.4) (end 96.76 78.4) (stroke (width 0.1) (type default)) (layer "Edge.Cuts"))
 (gr_line (start 118.76 154.4) (end 118.76 78.4) (stroke (width 0.1) (type default)) (layer "Edge.Cuts"))
 (gr_line (start 96.76 78.4) (end 96.76 154.4) (stroke (width 0.1) (type default)) (layer "Edge.Cuts"))
 (via (at 112.76 154.63) (size 0.6) (drill 0.3) (layers "F.Cu" "B.Cu") (free yes) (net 5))
 (segment (start 112.76 154.63) (end 112.76 157) (width 0.2) (layer "B.Cu") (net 5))
 (segment (start 101.11 154.295001) (end 101.11 153.95) (width 0.2) (layer "F.Cu") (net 42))
 (segment (start 101.01 157.25) (end 101.01 155.974999) (width 0.2) (layer "F.Cu") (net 42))
 (segment (start 100.985 154.420001) (end 101.11 154.295001) (width 0.2) (layer "F.Cu") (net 42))
 (segment (start 100.985 155.949999) (end 100.985 154.420001) (width 0.2) (layer "F.Cu") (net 42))
 (segment (start 101.01 155.974999) (end 100.985 155.949999) (width 0.2) (layer "F.Cu") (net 42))
 (segment (start 106.535 155.949999) (end 106.535 154.420001) (width 0.2) (layer "F.Cu") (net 1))
 (segment (start 106.51 157.25) (end 106.51 155.974999) (width 0.2) (layer "F.Cu") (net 1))
 (segment (start 106.41 154.295001) (end 106.41 153.95) (width 0.2) (layer "F.Cu") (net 1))
 (segment (start 106.51 155.974999) (end 106.535 155.949999) (width 0.2) (layer "F.Cu") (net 1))
 (segment (start 106.535 154.420001) (end 106.41 154.295001) (width 0.2) (layer "F.Cu") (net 1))
 (segment (start 100.51 155.974999) (end 100.535 155.949999) (width 0.2) (layer "F.Cu") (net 44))
 (segment (start 100.51 157.25) (end 100.51 155.974999) (width 0.2) (layer "F.Cu") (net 44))
 (segment (start 100.535 155.949999) (end 100.535 154.420001) (width 0.2) (layer "F.Cu") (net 44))
 (segment (start 100.535 154.420001) (end 100.41 154.295001) (width 0.2) (layer "F.Cu") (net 44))
 (segment (start 100.41 154.295001) (end 100.41 153.95) (width 0.2) (layer "F.Cu") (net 44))
 (segment (start 107.01 155.974999) (end 106.985 155.949999) (width 0.2) (layer "F.Cu") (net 3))
 (segment (start 107.11 154.295001) (end 107.11 153.95) (width 0.2) (layer "F.Cu") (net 3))
 (segment (start 106.985 154.420001) (end 107.11 154.295001) (width 0.2) (layer "F.Cu") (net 3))
 (segment (start 106.985 155.949999) (end 106.985 154.420001) (width 0.2) (layer "F.Cu") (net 3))
 (segment (start 107.01 157.25) (end 107.01 155.974999) (width 0.2) (layer "F.Cu") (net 3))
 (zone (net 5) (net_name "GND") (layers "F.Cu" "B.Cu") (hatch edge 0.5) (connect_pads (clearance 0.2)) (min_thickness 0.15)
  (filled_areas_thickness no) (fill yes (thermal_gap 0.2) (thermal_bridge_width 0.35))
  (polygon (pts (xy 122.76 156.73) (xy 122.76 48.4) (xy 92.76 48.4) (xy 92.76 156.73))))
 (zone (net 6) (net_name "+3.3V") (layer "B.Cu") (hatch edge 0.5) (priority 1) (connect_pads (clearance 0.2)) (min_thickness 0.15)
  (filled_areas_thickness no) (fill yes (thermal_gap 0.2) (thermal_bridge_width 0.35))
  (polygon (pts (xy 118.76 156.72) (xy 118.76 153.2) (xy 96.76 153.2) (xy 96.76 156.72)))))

